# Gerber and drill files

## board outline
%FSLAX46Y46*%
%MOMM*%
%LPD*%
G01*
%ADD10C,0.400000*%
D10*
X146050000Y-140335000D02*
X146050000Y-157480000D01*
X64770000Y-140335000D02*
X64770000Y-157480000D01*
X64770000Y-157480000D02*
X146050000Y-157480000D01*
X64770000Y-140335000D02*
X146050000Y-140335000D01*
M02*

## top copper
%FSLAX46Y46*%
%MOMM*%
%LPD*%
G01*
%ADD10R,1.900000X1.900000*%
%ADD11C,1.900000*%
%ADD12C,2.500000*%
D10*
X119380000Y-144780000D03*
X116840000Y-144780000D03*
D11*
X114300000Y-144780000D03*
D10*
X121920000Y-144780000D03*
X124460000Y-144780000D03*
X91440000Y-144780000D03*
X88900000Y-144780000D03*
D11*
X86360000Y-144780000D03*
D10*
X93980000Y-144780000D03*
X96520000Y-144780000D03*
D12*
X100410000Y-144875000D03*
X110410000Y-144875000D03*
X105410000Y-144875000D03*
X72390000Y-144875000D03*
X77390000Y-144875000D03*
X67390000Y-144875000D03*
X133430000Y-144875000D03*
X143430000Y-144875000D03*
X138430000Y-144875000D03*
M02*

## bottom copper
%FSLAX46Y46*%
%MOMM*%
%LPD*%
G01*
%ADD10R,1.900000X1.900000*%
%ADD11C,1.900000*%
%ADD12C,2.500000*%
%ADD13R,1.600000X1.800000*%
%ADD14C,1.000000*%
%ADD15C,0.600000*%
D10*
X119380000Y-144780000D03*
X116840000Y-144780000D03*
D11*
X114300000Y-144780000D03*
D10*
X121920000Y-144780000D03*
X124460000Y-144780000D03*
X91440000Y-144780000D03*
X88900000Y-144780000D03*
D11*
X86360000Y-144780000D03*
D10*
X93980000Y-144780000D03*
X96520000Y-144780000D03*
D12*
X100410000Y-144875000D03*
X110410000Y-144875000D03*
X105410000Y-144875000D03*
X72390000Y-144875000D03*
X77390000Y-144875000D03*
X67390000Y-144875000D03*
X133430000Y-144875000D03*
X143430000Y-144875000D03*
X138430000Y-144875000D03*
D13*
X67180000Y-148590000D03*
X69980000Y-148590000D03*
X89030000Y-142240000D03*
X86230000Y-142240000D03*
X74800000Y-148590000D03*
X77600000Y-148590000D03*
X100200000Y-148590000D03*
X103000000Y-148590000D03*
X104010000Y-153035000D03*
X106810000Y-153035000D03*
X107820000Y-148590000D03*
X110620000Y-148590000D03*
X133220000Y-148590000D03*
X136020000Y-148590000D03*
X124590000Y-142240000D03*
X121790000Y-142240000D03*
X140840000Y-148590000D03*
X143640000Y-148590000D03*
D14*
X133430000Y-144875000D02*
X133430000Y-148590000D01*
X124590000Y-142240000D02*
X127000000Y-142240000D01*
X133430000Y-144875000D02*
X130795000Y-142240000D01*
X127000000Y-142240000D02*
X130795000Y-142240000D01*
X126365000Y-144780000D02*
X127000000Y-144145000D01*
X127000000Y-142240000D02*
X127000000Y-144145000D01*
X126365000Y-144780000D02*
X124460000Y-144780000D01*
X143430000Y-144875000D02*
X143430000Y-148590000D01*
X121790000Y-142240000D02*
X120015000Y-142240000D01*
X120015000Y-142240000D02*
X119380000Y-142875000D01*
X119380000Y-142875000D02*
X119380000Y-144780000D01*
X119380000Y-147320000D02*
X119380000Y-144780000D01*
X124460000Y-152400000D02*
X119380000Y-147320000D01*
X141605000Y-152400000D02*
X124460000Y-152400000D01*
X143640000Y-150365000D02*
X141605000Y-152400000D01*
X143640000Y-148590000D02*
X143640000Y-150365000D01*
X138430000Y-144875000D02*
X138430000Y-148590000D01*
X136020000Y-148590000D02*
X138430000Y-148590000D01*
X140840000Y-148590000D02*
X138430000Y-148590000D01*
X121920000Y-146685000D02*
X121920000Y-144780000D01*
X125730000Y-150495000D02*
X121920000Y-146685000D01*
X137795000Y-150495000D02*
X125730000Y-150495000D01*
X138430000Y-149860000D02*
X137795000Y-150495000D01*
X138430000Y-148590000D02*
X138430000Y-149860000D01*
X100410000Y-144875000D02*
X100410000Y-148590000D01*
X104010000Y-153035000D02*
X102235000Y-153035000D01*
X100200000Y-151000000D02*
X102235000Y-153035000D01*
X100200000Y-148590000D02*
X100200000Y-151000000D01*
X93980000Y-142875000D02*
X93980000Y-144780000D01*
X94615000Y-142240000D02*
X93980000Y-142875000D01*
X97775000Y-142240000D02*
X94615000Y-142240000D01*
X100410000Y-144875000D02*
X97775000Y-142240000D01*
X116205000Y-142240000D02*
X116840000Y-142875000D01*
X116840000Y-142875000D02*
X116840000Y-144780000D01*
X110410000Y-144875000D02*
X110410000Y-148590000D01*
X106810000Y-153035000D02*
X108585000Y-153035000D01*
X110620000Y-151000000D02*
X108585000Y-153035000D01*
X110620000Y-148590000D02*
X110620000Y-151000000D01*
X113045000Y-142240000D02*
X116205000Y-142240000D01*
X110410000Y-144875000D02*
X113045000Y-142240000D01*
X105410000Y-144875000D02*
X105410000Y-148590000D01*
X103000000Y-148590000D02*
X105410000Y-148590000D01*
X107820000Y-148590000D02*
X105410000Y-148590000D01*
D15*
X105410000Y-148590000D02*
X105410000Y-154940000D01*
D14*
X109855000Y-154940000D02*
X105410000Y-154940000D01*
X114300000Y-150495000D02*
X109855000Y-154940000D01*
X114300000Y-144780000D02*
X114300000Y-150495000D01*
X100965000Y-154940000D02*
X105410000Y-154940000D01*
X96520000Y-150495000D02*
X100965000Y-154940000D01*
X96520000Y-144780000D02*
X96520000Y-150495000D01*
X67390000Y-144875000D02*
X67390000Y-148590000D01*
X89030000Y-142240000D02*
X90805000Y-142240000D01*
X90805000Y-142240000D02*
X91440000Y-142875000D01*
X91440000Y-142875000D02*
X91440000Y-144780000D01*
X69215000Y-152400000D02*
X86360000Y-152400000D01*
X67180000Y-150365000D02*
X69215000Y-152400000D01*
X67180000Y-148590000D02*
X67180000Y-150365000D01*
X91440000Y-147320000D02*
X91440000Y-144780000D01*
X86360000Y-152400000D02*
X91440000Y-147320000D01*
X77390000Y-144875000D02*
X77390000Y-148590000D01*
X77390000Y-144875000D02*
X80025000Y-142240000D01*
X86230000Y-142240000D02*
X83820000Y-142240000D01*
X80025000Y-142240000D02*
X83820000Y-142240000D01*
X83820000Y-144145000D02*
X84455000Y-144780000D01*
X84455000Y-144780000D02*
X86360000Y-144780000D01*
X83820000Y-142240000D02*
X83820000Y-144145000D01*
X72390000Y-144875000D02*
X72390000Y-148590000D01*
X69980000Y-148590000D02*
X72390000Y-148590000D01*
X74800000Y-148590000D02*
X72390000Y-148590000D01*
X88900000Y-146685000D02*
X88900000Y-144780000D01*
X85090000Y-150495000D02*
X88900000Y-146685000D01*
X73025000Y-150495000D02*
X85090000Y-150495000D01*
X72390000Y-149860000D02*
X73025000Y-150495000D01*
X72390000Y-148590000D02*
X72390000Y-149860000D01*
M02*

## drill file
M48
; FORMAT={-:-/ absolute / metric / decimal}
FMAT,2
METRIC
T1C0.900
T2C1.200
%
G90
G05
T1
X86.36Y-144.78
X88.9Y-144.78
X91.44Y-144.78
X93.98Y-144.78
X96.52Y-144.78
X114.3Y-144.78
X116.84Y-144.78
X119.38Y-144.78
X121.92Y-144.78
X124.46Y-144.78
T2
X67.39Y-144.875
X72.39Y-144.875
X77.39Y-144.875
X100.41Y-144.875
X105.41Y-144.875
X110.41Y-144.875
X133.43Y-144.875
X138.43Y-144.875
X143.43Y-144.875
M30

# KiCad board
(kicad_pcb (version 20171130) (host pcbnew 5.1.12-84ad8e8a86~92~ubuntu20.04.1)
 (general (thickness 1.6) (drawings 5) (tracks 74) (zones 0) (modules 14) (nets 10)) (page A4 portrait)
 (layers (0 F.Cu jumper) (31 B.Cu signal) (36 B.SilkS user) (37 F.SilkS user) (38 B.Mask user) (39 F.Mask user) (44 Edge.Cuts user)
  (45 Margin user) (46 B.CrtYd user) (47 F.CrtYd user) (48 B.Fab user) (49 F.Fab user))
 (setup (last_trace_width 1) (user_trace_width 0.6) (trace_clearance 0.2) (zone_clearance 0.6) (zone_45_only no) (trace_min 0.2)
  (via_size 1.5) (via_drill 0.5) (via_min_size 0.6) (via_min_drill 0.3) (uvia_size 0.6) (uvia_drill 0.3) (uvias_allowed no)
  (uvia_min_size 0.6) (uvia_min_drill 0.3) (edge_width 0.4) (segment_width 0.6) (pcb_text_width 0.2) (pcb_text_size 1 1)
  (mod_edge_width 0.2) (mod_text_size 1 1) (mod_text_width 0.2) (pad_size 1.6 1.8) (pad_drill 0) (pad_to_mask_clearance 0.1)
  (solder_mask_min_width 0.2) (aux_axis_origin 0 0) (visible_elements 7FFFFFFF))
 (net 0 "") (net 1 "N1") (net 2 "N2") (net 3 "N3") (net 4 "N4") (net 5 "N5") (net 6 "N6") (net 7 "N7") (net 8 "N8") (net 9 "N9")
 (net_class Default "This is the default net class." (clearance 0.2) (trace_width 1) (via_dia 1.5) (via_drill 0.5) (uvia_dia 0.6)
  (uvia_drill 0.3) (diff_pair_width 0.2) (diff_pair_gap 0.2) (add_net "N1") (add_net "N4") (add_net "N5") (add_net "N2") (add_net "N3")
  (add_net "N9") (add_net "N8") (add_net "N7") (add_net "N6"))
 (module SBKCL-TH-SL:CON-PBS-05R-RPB (layer F.Cu) (at 119.38 144.78)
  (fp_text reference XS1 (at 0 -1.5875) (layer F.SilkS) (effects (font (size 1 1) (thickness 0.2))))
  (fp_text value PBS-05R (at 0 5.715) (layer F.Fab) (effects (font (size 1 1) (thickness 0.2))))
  (pad 3 thru_hole rect (at 0 0) (size 1.9 1.9) (drill 0.9) (layers B.Cu B.Mask) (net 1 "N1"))
  (pad 2 thru_hole rect (at -2.54 0) (size 1.9 1.9) (drill 0.9) (layers B.Cu B.Mask) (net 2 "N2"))
  (pad 1 thru_hole circle (at -5.08 0) (size 1.9 1.9) (drill 0.9) (layers B.Cu B.Mask) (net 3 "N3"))
  (pad 4 thru_hole rect (at 2.54 0) (size 1.9 1.9) (drill 0.9) (layers B.Cu B.Mask) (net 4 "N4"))
  (pad 5 thru_hole rect (at 5.08 0) (size 1.9 1.9) (drill 0.9) (layers B.Cu B.Mask) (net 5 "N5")))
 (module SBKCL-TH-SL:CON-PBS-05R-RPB (layer F.Cu) (at 91.44 144.78)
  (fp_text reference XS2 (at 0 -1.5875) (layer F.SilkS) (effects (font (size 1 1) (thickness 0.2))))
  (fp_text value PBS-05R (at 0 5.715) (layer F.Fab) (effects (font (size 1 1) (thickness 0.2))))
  (pad 3 thru_hole rect (at 0 0) (size 1.9 1.9) (drill 0.9) (layers B.Cu B.Mask) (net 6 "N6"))
  (pad 2 thru_hole rect (at -2.54 0) (size 1.9 1.9) (drill 0.9) (layers B.Cu B.Mask) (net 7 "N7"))
  (pad 1 thru_hole circle (at -5.08 0) (size 1.9 1.9) (drill 0.9) (layers B.Cu B.Mask) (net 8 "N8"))
  (pad 4 thru_hole rect (at 2.54 0) (size 1.9 1.9) (drill 0.9) (layers B.Cu B.Mask) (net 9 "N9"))
  (pad 5 thru_hole rect (at 5.08 0) (size 1.9 1.9) (drill 0.9) (layers B.Cu B.Mask) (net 3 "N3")))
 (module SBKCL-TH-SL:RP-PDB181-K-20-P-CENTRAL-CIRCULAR (layer F.Cu) (at 105.41 144.875 180)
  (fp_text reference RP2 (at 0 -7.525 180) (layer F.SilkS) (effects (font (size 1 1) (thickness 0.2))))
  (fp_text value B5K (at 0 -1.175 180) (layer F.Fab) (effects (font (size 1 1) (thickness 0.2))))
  (pad 3 thru_hole circle (at 5 0 180) (size 2.5 2.5) (drill 1.2) (layers B.Cu B.Mask) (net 9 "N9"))
  (pad 1 thru_hole circle (at -5 0 180) (size 2.5 2.5) (drill 1.2) (layers B.Cu B.Mask) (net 2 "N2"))
  (pad 2 thru_hole circle (at 0 0 180) (size 2.5 2.5) (drill 1.2) (layers B.Cu B.Mask) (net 3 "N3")))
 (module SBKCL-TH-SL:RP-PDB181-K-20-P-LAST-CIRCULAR (layer F.Cu) (at 72.39 144.875 180)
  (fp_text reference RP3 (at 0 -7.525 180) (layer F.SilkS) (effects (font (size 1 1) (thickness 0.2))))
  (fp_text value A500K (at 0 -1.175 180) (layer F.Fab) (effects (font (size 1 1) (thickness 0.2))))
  (pad 2 thru_hole circle (at 0 0 180) (size 2.5 2.5) (drill 1.2) (layers B.Cu B.Mask) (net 7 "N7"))
  (pad 1 thru_hole circle (at -5 0 180) (size 2.5 2.5) (drill 1.2) (layers B.Cu B.Mask) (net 8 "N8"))
  (pad 3 thru_hole circle (at 5 0 180) (size 2.5 2.5) (drill 1.2) (layers B.Cu B.Mask) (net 6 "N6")))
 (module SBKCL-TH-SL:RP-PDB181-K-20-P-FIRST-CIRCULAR (layer F.Cu) (at 138.43 144.875 180)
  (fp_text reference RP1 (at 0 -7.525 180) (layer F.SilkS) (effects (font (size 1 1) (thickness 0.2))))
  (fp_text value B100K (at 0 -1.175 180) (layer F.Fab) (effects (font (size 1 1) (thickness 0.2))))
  (pad 3 thru_hole circle (at 5 0 180) (size 2.5 2.5) (drill 1.2) (layers B.Cu B.Mask) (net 5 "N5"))
  (pad 1 thru_hole circle (at -5 0 180) (size 2.5 2.5) (drill 1.2) (layers B.Cu B.Mask) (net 1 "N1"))
  (pad 2 thru_hole circle (at 0 0 180) (size 2.5 2.5) (drill 1.2) (layers B.Cu B.Mask) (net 4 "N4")))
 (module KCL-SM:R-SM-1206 (layer B.Cu) (at 68.58 148.59)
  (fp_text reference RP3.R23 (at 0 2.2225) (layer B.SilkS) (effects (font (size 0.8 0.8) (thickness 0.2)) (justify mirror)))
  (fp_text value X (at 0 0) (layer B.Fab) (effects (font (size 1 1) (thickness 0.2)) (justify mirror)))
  (pad 1 smd rect (at -1.4 0) (size 1.6 1.8) (layers B.Cu B.Mask) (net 6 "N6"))
  (pad 2 smd rect (at 1.4 0) (size 1.6 1.8) (layers B.Cu B.Mask) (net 7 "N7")))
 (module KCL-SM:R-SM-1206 (layer B.Cu) (at 87.63 142.24 180)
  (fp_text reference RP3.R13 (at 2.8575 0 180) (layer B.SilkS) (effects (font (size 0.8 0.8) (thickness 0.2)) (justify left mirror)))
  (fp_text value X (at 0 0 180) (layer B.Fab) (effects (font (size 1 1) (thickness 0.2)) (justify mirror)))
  (pad 1 smd rect (at -1.4 0 180) (size 1.6 1.8) (layers B.Cu B.Mask) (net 6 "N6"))
  (pad 2 smd rect (at 1.4 0 180) (size 1.6 1.8) (layers B.Cu B.Mask) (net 8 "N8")))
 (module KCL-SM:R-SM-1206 (layer B.Cu) (at 76.2 148.59)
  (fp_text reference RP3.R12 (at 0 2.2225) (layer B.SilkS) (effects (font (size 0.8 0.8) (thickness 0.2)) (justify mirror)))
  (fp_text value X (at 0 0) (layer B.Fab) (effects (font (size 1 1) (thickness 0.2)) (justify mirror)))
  (pad 1 smd rect (at -1.4 0) (size 1.6 1.8) (layers B.Cu B.Mask) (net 7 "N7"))
  (pad 2 smd rect (at 1.4 0) (size 1.6 1.8) (layers B.Cu B.Mask) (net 8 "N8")))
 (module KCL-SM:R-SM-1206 (layer B.Cu) (at 101.6 148.59)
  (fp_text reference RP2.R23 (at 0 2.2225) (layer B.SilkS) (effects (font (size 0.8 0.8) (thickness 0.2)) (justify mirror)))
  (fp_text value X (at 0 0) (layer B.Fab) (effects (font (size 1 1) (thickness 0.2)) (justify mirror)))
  (pad 1 smd rect (at -1.4 0) (size 1.6 1.8) (layers B.Cu B.Mask) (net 9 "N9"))
  (pad 2 smd rect (at 1.4 0) (size 1.6 1.8) (layers B.Cu B.Mask) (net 3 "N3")))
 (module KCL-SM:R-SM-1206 (layer B.Cu) (at 105.41 153.035)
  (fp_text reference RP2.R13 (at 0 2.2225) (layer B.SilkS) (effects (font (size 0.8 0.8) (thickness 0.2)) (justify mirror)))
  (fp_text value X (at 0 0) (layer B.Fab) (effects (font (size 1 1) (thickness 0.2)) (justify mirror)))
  (pad 1 smd rect (at -1.4 0) (size 1.6 1.8) (layers B.Cu B.Mask) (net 9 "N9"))
  (pad 2 smd rect (at 1.4 0) (size 1.6 1.8) (layers B.Cu B.Mask) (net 2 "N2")))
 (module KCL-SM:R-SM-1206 (layer B.Cu) (at 109.22 148.59)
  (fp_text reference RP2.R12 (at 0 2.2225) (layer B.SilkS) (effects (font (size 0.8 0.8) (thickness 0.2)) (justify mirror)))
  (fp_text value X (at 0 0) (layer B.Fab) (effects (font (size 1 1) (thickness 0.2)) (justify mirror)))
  (pad 1 smd rect (at -1.4 0) (size 1.6 1.8) (layers B.Cu B.Mask) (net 3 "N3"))
  (pad 2 smd rect (at 1.4 0) (size 1.6 1.8) (layers B.Cu B.Mask) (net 2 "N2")))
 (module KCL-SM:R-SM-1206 (layer B.Cu) (at 134.62 148.59)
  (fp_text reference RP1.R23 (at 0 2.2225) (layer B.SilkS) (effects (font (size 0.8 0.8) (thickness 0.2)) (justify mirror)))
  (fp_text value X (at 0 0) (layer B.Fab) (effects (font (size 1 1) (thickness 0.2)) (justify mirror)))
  (pad 1 smd rect (at -1.4 0) (size 1.6 1.8) (layers B.Cu B.Mask) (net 5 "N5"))
  (pad 2 smd rect (at 1.4 0) (size 1.6 1.8) (layers B.Cu B.Mask) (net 4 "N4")))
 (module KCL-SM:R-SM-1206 (layer B.Cu) (at 123.19 142.24 180)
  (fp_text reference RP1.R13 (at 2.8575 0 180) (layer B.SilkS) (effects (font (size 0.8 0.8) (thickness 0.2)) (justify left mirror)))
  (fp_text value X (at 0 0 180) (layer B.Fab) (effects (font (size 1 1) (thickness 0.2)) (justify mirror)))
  (pad 1 smd rect (at -1.4 0 180) (size 1.6 1.8) (layers B.Cu B.Mask) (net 5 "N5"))
  (pad 2 smd rect (at 1.4 0 180) (size 1.6 1.8) (layers B.Cu B.Mask) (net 1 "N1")))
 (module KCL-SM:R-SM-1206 (layer B.Cu) (at 142.24 148.59)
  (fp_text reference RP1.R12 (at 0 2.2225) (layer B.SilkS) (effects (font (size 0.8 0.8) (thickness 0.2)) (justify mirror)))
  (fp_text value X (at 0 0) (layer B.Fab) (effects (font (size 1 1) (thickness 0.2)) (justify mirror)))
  (pad 1 smd rect (at -1.4 0) (size 1.6 1.8) (layers B.Cu B.Mask) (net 4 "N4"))
  (pad 2 smd rect (at 1.4 0) (size 1.6 1.8) (layers B.Cu B.Mask) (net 1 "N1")))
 (gr_line (start 146.05 140.335) (end 146.05 157.48) (layer Edge.Cuts) (width 0.4))
 (gr_line (start 64.77 140.335) (end 64.77 157.48) (layer Edge.Cuts) (width 0.4))
 (gr_line (start 64.77 157.48) (end 146.05 157.48) (layer Edge.Cuts) (width 0.4))
 (gr_line (start 64.77 140.335) (end 146.05 140.335) (layer Edge.Cuts) (width 0.4))
 (segment (start 133.43 144.875) (end 133.43 148.59) (width 1) (layer B.Cu) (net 5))
 (segment (start 124.59 142.24) (end 127 142.24) (width 1) (layer B.Cu) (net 5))
 (segment (start 133.43 144.875) (end 130.795 142.24) (width 1) (layer B.Cu) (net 5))
 (segment (start 127 142.24) (end 130.795 142.24) (width 1) (layer B.Cu) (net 5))
 (segment (start 126.365 144.78) (end 127 144.145) (width 1) (layer B.Cu) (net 5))
 (segment (start 127 142.24) (end 127 144.145) (width 1) (layer B.Cu) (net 5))
 (segment (start 126.365 144.78) (end 124.46 144.78) (width 1) (layer B.Cu) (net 5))
 (segment (start 143.43 144.875) (end 143.43 148.59) (width 1) (layer B.Cu) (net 1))
 (segment (start 121.79 142.24) (end 120.015 142.24) (width 1) (layer B.Cu) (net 1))
 (segment (start 120.015 142.24) (end 119.38 142.875) (width 1) (layer B.Cu) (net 1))
 (segment (start 119.38 142.875) (end 119.38 144.78) (width 1) (layer B.Cu) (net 1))
 (segment (start 119.38 147.32) (end 119.38 144.78) (width 1) (layer B.Cu) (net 1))
 (segment (start 124.46 152.4) (end 119.38 147.32) (width 1) (layer B.Cu) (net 1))
 (segment (start 141.605 152.4) (end 124.46 152.4) (width 1) (layer B.Cu) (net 1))
 (segment (start 143.64 150.365) (end 141.605 152.4) (width 1) (layer B.Cu) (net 1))
 (segment (start 143.64 148.59) (end 143.64 150.365) (width 1) (layer B.Cu) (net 1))
 (segment (start 138.43 144.875) (end 138.43 148.59) (width 1) (layer B.Cu) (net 4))
 (segment (start 136.02 148.59) (end 138.43 148.59) (width 1) (layer B.Cu) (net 4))
 (segment (start 140.84 148.59) (end 138.43 148.59) (width 1) (layer B.Cu) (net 4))
 (segment (start 121.92 146.685) (end 121.92 144.78) (width 1) (layer B.Cu) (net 4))
 (segment (start 125.73 150.495) (end 121.92 146.685) (width 1) (layer B.Cu) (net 4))
 (segment (start 137.795 150.495) (end 125.73 150.495) (width 1) (layer B.Cu) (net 4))
 (segment (start 138.43 149.86) (end 137.795 150.495) (width 1) (layer B.Cu) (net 4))
 (segment (start 138.43 148.59) (end 138.43 149.86) (width 1) (layer B.Cu) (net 4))
 (segment (start 100.41 144.875) (end 100.41 148.59) (width 1) (layer B.Cu) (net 9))
 (segment (start 104.01 153.035) (end 102.235 153.035) (width 1) (layer B.Cu) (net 9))
 (segment (start 100.2 151) (end 102.235 153.035) (width 1) (layer B.Cu) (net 9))
 (segment (start 100.2 148.59) (end 100.2 151) (width 1) (layer B.Cu) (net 9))
 (segment (start 93.98 142.875) (end 93.98 144.78) (width 1) (layer B.Cu) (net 9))
 (segment (start 94.615 142.24) (end 93.98 142.875) (width 1) (layer B.Cu) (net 9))
 (segment (start 97.775 142.24) (end 94.615 142.24) (width 1) (layer B.Cu) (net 9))
 (segment (start 100.41 144.875) (end 97.775 142.24) (width 1) (layer B.Cu) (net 9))
 (segment (start 116.205 142.24) (end 116.84 142.875) (width 1) (layer B.Cu) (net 2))
 (segment (start 116.84 142.875) (end 116.84 144.78) (width 1) (layer B.Cu) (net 2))
 (segment (start 110.41 144.875) (end 110.41 148.59) (width 1) (layer B.Cu) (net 2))
 (segment (start 106.81 153.035) (end 108.585 153.035) (width 1) (layer B.Cu) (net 2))
 (segment (start 110.62 151) (end 108.585 153.035) (width 1) (layer B.Cu) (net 2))
 (segment (start 110.62 148.59) (end 110.62 151) (width 1) (layer B.Cu) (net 2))
 (segment (start 113.045 142.24) (end 116.205 142.24) (width 1) (layer B.Cu) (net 2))
 (segment (start 110.41 144.875) (end 113.045 142.24) (width 1) (layer B.Cu) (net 2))
 (segment (start 105.41 144.875) (end 105.41 148.59) (width 1) (layer B.Cu) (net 3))
 (segment (start 103 148.59) (end 105.41 148.59) (width 1) (layer B.Cu) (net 3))
 (segment (start 107.82 148.59) (end 105.41 148.59) (width 1) (layer B.Cu) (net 3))
 (segment (start 105.41 148.59) (end 105.41 154.94) (width 0.6) (layer B.Cu) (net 3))
 (segment (start 109.855 154.94) (end 105.41 154.94) (width 1) (layer B.Cu) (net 3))
 (segment (start 114.3 150.495) (end 109.855 154.94) (width 1) (layer B.Cu) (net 3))
 (segment (start 114.3 144.78) (end 114.3 150.495) (width 1) (layer B.Cu) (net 3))
 (segment (start 100.965 154.94) (end 105.41 154.94) (width 1) (layer B.Cu) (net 3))
 (segment (start 96.52 150.495) (end 100.965 154.94) (width 1) (layer B.Cu) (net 3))
 (segment (start 96.52 144.78) (end 96.52 150.495) (width 1) (layer B.Cu) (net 3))
 (segment (start 67.39 144.875) (end 67.39 148.59) (width 1) (layer B.Cu) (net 6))
 (segment (start 89.03 142.24) (end 90.805 142.24) (width 1) (layer B.Cu) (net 6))
 (segment (start 90.805 142.24) (end 91.44 142.875) (width 1) (layer B.Cu) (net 6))
 (segment (start 91.44 142.875) (end 91.44 144.78) (width 1) (layer B.Cu) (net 6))
 (segment (start 69.215 152.4) (end 86.36 152.4) (width 1) (layer B.Cu) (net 6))
 (segment (start 67.18 150.365) (end 69.215 152.4) (width 1) (layer B.Cu) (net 6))
 (segment (start 67.18 148.59) (end 67.18 150.365) (width 1) (layer B.Cu) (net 6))
 (segment (start 91.44 147.32) (end 91.44 144.78) (width 1) (layer B.Cu) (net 6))
 (segment (start 86.36 152.4) (end 91.44 147.32) (width 1) (layer B.Cu) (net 6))
 (segment (start 77.39 144.875) (end 77.39 148.59) (width 1) (layer B.Cu) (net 8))
 (segment (start 77.39 144.875) (end 80.025 142.24) (width 1) (layer B.Cu) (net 8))
 (segment (start 86.23 142.24) (end 83.82 142.24) (width 1) (layer B.Cu) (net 8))
 (segment (start 80.025 142.24) (end 83.82 142.24) (width 1) (layer B.Cu) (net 8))
 (segment (start 83.82 144.145) (end 84.455 144.78) (width 1) (layer B.Cu) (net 8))
 (segment (start 84.455 144.78) (end 86.36 144.78) (width 1) (layer B.Cu) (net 8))
 (segment (start 83.82 142.24) (end 83.82 144.145) (width 1) (layer B.Cu) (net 8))
 (segment (start 72.39 144.875) (end 72.39 148.59) (width 1) (layer B.Cu) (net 7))
 (segment (start 69.98 148.59) (end 72.39 148.59) (width 1) (layer B.Cu) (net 7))
 (segment (start 74.8 148.59) (end 72.39 148.59) (width 1) (layer B.Cu) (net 7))
 (segment (start 88.9 146.685) (end 88.9 144.78) (width 1) (layer B.Cu) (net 7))
 (segment (start 85.09 150.495) (end 88.9 146.685) (width 1) (layer B.Cu) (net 7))
 (segment (start 73.025 150.495) (end 85.09 150.495) (width 1) (layer B.Cu) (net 7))
 (segment (start 72.39 149.86) (end 73.025 150.495) (width 1) (layer B.Cu) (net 7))
 (segment (start 72.39 148.59) (end 72.39 149.86) (width 1) (layer B.Cu) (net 7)))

